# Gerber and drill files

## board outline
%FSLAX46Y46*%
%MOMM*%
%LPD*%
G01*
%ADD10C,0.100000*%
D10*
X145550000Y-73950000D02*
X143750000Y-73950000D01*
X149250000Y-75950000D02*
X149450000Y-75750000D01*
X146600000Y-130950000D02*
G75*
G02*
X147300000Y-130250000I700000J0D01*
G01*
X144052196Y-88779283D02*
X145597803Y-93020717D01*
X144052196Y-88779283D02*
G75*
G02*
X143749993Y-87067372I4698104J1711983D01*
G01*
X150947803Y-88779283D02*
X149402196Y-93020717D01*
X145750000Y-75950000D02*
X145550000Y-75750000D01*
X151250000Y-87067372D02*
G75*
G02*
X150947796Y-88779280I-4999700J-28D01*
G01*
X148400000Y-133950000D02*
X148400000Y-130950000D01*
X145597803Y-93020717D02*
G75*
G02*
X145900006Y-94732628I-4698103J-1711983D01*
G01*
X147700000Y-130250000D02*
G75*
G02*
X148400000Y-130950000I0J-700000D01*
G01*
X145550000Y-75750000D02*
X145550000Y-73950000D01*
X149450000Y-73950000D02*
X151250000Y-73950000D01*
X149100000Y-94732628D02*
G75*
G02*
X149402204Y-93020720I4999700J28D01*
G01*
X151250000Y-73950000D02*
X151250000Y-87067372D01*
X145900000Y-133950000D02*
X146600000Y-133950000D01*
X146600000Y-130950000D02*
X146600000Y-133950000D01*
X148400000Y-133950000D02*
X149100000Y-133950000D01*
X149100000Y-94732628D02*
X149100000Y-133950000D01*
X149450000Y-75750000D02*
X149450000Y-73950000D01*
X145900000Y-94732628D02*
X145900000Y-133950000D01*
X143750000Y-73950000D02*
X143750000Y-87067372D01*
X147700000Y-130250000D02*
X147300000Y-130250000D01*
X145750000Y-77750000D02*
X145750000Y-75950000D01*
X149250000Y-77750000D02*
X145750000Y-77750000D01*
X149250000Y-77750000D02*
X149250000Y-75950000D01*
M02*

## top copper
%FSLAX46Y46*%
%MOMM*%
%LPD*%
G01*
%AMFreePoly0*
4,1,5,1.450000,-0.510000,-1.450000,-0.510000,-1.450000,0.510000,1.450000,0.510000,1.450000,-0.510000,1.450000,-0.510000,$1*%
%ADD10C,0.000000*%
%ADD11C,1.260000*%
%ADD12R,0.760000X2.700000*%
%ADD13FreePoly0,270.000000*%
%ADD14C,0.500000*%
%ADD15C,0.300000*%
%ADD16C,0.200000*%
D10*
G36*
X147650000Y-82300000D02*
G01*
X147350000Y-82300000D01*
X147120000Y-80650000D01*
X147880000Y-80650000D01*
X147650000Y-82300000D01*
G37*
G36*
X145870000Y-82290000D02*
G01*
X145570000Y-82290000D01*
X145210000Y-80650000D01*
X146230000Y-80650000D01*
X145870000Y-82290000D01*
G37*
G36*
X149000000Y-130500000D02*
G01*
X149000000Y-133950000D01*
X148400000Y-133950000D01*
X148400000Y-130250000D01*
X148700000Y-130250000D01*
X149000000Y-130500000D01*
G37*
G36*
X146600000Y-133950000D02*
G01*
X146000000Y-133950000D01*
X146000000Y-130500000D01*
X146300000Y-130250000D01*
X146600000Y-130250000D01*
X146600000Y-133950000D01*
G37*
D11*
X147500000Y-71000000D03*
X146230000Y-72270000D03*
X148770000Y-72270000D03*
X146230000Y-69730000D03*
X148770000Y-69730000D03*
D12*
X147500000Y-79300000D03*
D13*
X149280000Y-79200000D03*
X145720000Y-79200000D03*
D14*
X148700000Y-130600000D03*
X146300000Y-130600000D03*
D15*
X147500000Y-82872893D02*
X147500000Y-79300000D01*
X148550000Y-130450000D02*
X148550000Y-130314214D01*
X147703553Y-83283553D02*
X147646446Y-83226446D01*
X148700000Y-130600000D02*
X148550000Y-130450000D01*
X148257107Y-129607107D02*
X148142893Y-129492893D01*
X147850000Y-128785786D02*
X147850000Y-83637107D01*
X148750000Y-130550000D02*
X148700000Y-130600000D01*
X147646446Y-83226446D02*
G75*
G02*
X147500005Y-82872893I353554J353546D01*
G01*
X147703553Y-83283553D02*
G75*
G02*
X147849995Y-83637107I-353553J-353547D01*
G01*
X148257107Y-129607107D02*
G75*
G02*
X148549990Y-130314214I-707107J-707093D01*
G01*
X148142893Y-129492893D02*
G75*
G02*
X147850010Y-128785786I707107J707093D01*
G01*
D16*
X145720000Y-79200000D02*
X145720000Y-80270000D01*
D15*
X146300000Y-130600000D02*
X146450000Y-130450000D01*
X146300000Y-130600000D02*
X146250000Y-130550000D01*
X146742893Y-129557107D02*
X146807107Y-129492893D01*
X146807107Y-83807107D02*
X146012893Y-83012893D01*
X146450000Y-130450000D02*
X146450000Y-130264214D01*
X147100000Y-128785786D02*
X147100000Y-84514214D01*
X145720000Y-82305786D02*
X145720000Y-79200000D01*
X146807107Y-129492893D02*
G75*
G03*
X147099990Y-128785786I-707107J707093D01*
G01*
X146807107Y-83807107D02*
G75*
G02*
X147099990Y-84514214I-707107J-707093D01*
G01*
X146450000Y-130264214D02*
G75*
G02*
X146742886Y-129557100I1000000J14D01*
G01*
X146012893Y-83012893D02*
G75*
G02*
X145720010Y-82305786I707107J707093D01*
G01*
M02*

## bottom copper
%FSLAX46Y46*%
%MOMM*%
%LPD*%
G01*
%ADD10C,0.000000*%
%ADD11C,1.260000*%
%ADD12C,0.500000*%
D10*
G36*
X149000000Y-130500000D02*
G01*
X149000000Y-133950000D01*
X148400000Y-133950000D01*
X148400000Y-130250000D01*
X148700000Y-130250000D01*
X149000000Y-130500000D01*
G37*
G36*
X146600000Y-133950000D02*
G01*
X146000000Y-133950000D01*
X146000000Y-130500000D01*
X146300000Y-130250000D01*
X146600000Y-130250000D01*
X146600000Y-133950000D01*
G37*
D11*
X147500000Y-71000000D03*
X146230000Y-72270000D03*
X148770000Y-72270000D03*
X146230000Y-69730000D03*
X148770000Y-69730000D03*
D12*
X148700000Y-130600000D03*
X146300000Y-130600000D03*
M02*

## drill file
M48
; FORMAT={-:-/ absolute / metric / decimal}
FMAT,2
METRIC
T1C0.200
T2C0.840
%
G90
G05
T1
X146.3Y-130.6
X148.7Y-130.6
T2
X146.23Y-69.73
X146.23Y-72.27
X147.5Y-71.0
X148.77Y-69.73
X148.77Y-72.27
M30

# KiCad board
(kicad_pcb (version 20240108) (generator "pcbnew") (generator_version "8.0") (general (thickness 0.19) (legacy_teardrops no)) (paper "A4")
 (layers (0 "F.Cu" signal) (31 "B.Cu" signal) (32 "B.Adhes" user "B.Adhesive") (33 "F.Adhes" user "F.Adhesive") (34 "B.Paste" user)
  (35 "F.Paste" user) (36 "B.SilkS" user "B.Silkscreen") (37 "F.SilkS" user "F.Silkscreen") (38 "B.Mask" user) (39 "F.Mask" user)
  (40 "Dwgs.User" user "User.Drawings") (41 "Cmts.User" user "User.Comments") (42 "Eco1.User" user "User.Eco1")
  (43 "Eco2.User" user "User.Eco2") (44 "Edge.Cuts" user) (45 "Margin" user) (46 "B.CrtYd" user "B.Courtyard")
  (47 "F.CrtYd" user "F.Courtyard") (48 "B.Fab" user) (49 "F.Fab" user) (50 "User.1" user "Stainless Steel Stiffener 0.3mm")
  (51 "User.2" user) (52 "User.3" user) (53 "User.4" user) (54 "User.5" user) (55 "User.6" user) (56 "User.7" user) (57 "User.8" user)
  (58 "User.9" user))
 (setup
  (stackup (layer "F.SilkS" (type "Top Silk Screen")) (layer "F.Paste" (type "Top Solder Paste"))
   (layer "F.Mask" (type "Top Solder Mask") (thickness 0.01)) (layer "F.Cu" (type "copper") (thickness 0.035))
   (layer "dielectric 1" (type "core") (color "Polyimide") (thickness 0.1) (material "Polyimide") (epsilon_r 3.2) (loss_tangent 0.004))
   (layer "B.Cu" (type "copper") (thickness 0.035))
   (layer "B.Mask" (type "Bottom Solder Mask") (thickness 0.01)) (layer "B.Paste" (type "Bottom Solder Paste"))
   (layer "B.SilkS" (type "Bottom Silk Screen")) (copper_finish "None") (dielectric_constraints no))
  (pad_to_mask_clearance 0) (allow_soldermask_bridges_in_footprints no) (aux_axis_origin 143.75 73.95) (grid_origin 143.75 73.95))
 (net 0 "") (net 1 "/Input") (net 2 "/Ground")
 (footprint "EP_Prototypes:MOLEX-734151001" (layer "F.Cu") (at 147.5 71 90)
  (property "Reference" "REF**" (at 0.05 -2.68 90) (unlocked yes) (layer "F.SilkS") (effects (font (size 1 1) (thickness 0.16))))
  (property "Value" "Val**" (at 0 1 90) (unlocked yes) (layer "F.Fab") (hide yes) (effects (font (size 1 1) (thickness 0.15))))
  (pad "1" thru_hole circle (at 0 0 90) (size 1.26 1.26) (drill 0.84) (layers "*.Cu" "*.Mask") (remove_unused_layers no))
  (pad "2" thru_hole circle (at -1.27 -1.27 90) (size 1.26 1.26) (drill 0.84) (layers "*.Cu" "*.Mask") (remove_unused_layers no))
  (pad "2" thru_hole circle (at -1.27 1.27 90) (size 1.26 1.26) (drill 0.84) (layers "*.Cu" "*.Mask") (remove_unused_layers no))
  (pad "2" thru_hole circle (at 1.27 -1.27 90) (size 1.26 1.26) (drill 0.84) (layers "*.Cu" "*.Mask") (remove_unused_layers no))
  (pad "2" thru_hole circle (at 1.27 1.27 90) (size 1.26 1.26) (drill 0.84) (layers "*.Cu" "*.Mask") (remove_unused_layers no)))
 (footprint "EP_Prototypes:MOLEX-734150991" (layer "F.Cu") (at 147.5 77.76 -90)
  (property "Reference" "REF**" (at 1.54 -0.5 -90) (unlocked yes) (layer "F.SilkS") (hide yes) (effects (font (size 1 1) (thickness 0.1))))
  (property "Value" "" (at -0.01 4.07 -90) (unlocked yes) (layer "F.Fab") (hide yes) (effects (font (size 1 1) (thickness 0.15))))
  (fp_line (start -0.01 1.75) (end -1.81 1.75) (stroke (width 0.1) (type default)) (layer "Edge.Cuts"))
  (fp_line (start -0.01 -1.75) (end -0.01 1.75) (stroke (width 0.1) (type default)) (layer "Edge.Cuts"))
  (fp_line (start -0.01 -1.75) (end -1.81 -1.75) (stroke (width 0.1) (type default)) (layer "Edge.Cuts"))
  (pad "1" smd rect (at 1.54 0 270) (size 2.7 0.76) (layers "F.Cu" "F.Paste" "F.Mask") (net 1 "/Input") (thermal_bridge_angle 45))
  (pad "2" smd custom (at 1.44 -1.78 270) (size 2.9 1.02) (layers "F.Cu" "F.Paste" "F.Mask") (thermal_bridge_angle 45)
   (options (clearance outline) (anchor rect)) (primitives))
  (pad "2" smd custom (at 1.44 1.78 270) (size 2.9 1.02) (layers "F.Cu" "F.Paste" "F.Mask") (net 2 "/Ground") (thermal_bridge_angle 45)
   (options (clearance outline) (anchor rect)) (primitives)))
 (gr_poly
  (pts (xy 147.35 82.3) (xy 147.12 80.65) (xy 147.88 80.65) (xy 147.65 82.3)) (stroke (width 0) (type solid)) (fill solid) (layer "F.Cu")
  (net 1))
 (gr_poly
  (pts (xy 145.21 80.65) (xy 145.57 82.29) (xy 145.87 82.29) (xy 146.23 80.65)) (stroke (width 0) (type solid)) (fill solid) (layer "F.Cu")
  (net 2))
 (gr_poly
  (pts (xy 148.4 130.25) (xy 148.7 130.25) (xy 149 130.5) (xy 149 133.95) (xy 148.4 133.95)) (stroke (width 0) (type solid)) (fill solid)
  (layer "F.Cu") (net 1))
 (gr_poly
  (pts (xy 146.6 130.25) (xy 146.3 130.25) (xy 146 130.5) (xy 146 133.95) (xy 146.6 133.95)) (stroke (width 0) (type solid)) (fill solid)
  (layer "F.Cu") (net 2))
 (gr_poly
  (pts (xy 148.4 130.25) (xy 148.7 130.25) (xy 149 130.5) (xy 149 133.95) (xy 148.4 133.95)) (stroke (width 0) (type solid)) (fill solid)
  (layer "B.Cu") (net 1))
 (gr_poly
  (pts (xy 146.6 130.25) (xy 146.3 130.25) (xy 146 130.5) (xy 146 133.95) (xy 146.6 133.95)) (stroke (width 0) (type solid)) (fill solid)
  (layer "B.Cu") (net 2))
 (gr_line (start 145.55 73.95) (end 143.75 73.95) (stroke (width 0.1) (type default)) (layer "Edge.Cuts"))
 (gr_line (start 149.25 75.95) (end 149.45 75.75) (stroke (width 0.1) (type default)) (layer "Edge.Cuts"))
 (gr_arc (start 146.6 130.95) (mid 146.805025 130.455025) (end 147.3 130.25) (stroke (width 0.1) (type default)) (layer "Edge.Cuts"))
 (gr_line (start 144.052196 88.779283) (end 145.597803 93.020717) (stroke (width 0.1) (type default)) (layer "Edge.Cuts"))
 (gr_arc (start 144.052196 88.779283) (mid 143.826133 87.936561) (end 143.75 87.067372) (stroke (width 0.1) (type default))
  (layer "Edge.Cuts"))
 (gr_line (start 150.947803 88.779283) (end 149.402196 93.020717) (stroke (width 0.1) (type default)) (layer "Edge.Cuts"))
 (gr_line (start 145.75 75.95) (end 145.55 75.75) (stroke (width 0.1) (type default)) (layer "Edge.Cuts"))
 (gr_arc (start 151.25 87.067372) (mid 151.173876 87.936563) (end 150.947803 88.779283) (stroke (width 0.1) (type default))
  (layer "Edge.Cuts"))
 (gr_line (start 148.4 133.95) (end 148.4 130.95) (stroke (width 0.1) (type default)) (layer "Edge.Cuts"))
 (gr_arc (start 145.597803 93.020717) (mid 145.823866 93.863439) (end 145.9 94.732628) (stroke (width 0.1) (type default))
  (layer "Edge.Cuts"))
 (gr_arc (start 147.7 130.25) (mid 148.194975 130.455025) (end 148.4 130.95) (stroke (width 0.1) (type default)) (layer "Edge.Cuts"))
 (gr_line (start 145.55 75.75) (end 145.55 73.95) (stroke (width 0.1) (type default)) (layer "Edge.Cuts"))
 (gr_line (start 149.45 73.95) (end 151.25 73.95) (stroke (width 0.1) (type default)) (layer "Edge.Cuts"))
 (gr_arc (start 149.1 94.732628) (mid 149.176124 93.863437) (end 149.402196 93.020717) (stroke (width 0.1) (type default))
  (layer "Edge.Cuts"))
 (gr_line (start 151.25 73.95) (end 151.25 87.067372) (stroke (width 0.1) (type default)) (layer "Edge.Cuts"))
 (gr_line (start 145.9 133.95) (end 146.6 133.95) (stroke (width 0.1) (type default)) (layer "Edge.Cuts"))
 (gr_line (start 146.6 130.95) (end 146.6 133.95) (stroke (width 0.1) (type default)) (layer "Edge.Cuts"))
 (gr_line (start 148.4 133.95) (end 149.1 133.95) (stroke (width 0.1) (type default)) (layer "Edge.Cuts"))
 (gr_line (start 149.1 94.732628) (end 149.1 133.95) (stroke (width 0.1) (type default)) (layer "Edge.Cuts"))
 (gr_line (start 149.45 75.75) (end 149.45 73.95) (stroke (width 0.1) (type default)) (layer "Edge.Cuts"))
 (gr_line (start 145.9 94.732628) (end 145.9 133.95) (stroke (width 0.1) (type default)) (layer "Edge.Cuts"))
 (gr_line (start 143.75 73.95) (end 143.75 87.067372) (stroke (width 0.1) (type default)) (layer "Edge.Cuts"))
 (gr_line (start 147.7 130.25) (end 147.3 130.25) (stroke (width 0.1) (type default)) (layer "Edge.Cuts"))
 (segment (start 147.5 82.872893) (end 147.5 79.3) (width 0.3) (layer "F.Cu") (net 1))
 (segment (start 148.55 130.45) (end 148.55 130.314214) (width 0.3) (layer "F.Cu") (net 1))
 (segment (start 147.703553 83.283553) (end 147.646446 83.226446) (width 0.3) (layer "F.Cu") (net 1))
 (segment (start 148.7 130.6) (end 148.55 130.45) (width 0.3) (layer "F.Cu") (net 1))
 (segment (start 148.257107 129.607107) (end 148.142893 129.492893) (width 0.3) (layer "F.Cu") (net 1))
 (segment (start 147.85 128.785786) (end 147.85 83.637107) (width 0.3) (layer "F.Cu") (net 1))
 (segment (start 148.75 130.55) (end 148.7 130.6) (width 0.3) (layer "F.Cu") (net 1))
 (via (at 148.7 130.6) (size 0.5) (drill 0.2) (layers "F.Cu" "B.Cu") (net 1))
 (arc (start 147.646446 83.226446) (mid 147.53806 83.064234) (end 147.5 82.872893) (width 0.3) (layer "F.Cu") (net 1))
 (arc (start 147.703553 83.283553) (mid 147.81194 83.445765) (end 147.85 83.637107) (width 0.3) (layer "F.Cu") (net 1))
 (arc (start 148.257107 129.607107) (mid 148.47388 129.93153) (end 148.55 130.314214) (width 0.3) (layer "F.Cu") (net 1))
 (arc (start 148.142893 129.492893) (mid 147.92612 129.16847) (end 147.85 128.785786) (width 0.3) (layer "F.Cu") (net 1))
 (segment (start 145.72 79.2) (end 145.72 80.27) (width 0.2) (layer "F.Cu") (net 2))
 (segment (start 146.3 130.6) (end 146.45 130.45) (width 0.3) (layer "F.Cu") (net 2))
 (segment (start 146.3 130.6) (end 146.25 130.55) (width 0.3) (layer "F.Cu") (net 2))
 (segment (start 146.742893 129.557107) (end 146.807107 129.492893) (width 0.3) (layer "F.Cu") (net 2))
 (segment (start 146.807107 83.807107) (end 146.012893 83.012893) (width 0.3) (layer "F.Cu") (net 2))
 (segment (start 146.45 130.45) (end 146.45 130.264214) (width 0.3) (layer "F.Cu") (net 2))
 (segment (start 147.1 128.785786) (end 147.1 84.514214) (width 0.3) (layer "F.Cu") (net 2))
 (segment (start 145.72 82.305786) (end 145.72 79.2) (width 0.3) (layer "F.Cu") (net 2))
 (via (at 146.3 130.6) (size 0.5) (drill 0.2) (layers "F.Cu" "B.Cu") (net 2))
 (arc (start 146.807107 129.492893) (mid 147.02388 129.16847) (end 147.1 128.785786) (width 0.3) (layer "F.Cu") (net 2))
 (arc (start 146.807107 83.807107) (mid 147.02388 84.13153) (end 147.1 84.514214) (width 0.3) (layer "F.Cu") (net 2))
 (arc (start 146.45 130.264214) (mid 146.52612 129.881531) (end 146.742893 129.557107) (width 0.3) (layer "F.Cu") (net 2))
 (arc (start 146.012893 83.012893) (mid 145.79612 82.68847) (end 145.72 82.305786) (width 0.3) (layer "F.Cu") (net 2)))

